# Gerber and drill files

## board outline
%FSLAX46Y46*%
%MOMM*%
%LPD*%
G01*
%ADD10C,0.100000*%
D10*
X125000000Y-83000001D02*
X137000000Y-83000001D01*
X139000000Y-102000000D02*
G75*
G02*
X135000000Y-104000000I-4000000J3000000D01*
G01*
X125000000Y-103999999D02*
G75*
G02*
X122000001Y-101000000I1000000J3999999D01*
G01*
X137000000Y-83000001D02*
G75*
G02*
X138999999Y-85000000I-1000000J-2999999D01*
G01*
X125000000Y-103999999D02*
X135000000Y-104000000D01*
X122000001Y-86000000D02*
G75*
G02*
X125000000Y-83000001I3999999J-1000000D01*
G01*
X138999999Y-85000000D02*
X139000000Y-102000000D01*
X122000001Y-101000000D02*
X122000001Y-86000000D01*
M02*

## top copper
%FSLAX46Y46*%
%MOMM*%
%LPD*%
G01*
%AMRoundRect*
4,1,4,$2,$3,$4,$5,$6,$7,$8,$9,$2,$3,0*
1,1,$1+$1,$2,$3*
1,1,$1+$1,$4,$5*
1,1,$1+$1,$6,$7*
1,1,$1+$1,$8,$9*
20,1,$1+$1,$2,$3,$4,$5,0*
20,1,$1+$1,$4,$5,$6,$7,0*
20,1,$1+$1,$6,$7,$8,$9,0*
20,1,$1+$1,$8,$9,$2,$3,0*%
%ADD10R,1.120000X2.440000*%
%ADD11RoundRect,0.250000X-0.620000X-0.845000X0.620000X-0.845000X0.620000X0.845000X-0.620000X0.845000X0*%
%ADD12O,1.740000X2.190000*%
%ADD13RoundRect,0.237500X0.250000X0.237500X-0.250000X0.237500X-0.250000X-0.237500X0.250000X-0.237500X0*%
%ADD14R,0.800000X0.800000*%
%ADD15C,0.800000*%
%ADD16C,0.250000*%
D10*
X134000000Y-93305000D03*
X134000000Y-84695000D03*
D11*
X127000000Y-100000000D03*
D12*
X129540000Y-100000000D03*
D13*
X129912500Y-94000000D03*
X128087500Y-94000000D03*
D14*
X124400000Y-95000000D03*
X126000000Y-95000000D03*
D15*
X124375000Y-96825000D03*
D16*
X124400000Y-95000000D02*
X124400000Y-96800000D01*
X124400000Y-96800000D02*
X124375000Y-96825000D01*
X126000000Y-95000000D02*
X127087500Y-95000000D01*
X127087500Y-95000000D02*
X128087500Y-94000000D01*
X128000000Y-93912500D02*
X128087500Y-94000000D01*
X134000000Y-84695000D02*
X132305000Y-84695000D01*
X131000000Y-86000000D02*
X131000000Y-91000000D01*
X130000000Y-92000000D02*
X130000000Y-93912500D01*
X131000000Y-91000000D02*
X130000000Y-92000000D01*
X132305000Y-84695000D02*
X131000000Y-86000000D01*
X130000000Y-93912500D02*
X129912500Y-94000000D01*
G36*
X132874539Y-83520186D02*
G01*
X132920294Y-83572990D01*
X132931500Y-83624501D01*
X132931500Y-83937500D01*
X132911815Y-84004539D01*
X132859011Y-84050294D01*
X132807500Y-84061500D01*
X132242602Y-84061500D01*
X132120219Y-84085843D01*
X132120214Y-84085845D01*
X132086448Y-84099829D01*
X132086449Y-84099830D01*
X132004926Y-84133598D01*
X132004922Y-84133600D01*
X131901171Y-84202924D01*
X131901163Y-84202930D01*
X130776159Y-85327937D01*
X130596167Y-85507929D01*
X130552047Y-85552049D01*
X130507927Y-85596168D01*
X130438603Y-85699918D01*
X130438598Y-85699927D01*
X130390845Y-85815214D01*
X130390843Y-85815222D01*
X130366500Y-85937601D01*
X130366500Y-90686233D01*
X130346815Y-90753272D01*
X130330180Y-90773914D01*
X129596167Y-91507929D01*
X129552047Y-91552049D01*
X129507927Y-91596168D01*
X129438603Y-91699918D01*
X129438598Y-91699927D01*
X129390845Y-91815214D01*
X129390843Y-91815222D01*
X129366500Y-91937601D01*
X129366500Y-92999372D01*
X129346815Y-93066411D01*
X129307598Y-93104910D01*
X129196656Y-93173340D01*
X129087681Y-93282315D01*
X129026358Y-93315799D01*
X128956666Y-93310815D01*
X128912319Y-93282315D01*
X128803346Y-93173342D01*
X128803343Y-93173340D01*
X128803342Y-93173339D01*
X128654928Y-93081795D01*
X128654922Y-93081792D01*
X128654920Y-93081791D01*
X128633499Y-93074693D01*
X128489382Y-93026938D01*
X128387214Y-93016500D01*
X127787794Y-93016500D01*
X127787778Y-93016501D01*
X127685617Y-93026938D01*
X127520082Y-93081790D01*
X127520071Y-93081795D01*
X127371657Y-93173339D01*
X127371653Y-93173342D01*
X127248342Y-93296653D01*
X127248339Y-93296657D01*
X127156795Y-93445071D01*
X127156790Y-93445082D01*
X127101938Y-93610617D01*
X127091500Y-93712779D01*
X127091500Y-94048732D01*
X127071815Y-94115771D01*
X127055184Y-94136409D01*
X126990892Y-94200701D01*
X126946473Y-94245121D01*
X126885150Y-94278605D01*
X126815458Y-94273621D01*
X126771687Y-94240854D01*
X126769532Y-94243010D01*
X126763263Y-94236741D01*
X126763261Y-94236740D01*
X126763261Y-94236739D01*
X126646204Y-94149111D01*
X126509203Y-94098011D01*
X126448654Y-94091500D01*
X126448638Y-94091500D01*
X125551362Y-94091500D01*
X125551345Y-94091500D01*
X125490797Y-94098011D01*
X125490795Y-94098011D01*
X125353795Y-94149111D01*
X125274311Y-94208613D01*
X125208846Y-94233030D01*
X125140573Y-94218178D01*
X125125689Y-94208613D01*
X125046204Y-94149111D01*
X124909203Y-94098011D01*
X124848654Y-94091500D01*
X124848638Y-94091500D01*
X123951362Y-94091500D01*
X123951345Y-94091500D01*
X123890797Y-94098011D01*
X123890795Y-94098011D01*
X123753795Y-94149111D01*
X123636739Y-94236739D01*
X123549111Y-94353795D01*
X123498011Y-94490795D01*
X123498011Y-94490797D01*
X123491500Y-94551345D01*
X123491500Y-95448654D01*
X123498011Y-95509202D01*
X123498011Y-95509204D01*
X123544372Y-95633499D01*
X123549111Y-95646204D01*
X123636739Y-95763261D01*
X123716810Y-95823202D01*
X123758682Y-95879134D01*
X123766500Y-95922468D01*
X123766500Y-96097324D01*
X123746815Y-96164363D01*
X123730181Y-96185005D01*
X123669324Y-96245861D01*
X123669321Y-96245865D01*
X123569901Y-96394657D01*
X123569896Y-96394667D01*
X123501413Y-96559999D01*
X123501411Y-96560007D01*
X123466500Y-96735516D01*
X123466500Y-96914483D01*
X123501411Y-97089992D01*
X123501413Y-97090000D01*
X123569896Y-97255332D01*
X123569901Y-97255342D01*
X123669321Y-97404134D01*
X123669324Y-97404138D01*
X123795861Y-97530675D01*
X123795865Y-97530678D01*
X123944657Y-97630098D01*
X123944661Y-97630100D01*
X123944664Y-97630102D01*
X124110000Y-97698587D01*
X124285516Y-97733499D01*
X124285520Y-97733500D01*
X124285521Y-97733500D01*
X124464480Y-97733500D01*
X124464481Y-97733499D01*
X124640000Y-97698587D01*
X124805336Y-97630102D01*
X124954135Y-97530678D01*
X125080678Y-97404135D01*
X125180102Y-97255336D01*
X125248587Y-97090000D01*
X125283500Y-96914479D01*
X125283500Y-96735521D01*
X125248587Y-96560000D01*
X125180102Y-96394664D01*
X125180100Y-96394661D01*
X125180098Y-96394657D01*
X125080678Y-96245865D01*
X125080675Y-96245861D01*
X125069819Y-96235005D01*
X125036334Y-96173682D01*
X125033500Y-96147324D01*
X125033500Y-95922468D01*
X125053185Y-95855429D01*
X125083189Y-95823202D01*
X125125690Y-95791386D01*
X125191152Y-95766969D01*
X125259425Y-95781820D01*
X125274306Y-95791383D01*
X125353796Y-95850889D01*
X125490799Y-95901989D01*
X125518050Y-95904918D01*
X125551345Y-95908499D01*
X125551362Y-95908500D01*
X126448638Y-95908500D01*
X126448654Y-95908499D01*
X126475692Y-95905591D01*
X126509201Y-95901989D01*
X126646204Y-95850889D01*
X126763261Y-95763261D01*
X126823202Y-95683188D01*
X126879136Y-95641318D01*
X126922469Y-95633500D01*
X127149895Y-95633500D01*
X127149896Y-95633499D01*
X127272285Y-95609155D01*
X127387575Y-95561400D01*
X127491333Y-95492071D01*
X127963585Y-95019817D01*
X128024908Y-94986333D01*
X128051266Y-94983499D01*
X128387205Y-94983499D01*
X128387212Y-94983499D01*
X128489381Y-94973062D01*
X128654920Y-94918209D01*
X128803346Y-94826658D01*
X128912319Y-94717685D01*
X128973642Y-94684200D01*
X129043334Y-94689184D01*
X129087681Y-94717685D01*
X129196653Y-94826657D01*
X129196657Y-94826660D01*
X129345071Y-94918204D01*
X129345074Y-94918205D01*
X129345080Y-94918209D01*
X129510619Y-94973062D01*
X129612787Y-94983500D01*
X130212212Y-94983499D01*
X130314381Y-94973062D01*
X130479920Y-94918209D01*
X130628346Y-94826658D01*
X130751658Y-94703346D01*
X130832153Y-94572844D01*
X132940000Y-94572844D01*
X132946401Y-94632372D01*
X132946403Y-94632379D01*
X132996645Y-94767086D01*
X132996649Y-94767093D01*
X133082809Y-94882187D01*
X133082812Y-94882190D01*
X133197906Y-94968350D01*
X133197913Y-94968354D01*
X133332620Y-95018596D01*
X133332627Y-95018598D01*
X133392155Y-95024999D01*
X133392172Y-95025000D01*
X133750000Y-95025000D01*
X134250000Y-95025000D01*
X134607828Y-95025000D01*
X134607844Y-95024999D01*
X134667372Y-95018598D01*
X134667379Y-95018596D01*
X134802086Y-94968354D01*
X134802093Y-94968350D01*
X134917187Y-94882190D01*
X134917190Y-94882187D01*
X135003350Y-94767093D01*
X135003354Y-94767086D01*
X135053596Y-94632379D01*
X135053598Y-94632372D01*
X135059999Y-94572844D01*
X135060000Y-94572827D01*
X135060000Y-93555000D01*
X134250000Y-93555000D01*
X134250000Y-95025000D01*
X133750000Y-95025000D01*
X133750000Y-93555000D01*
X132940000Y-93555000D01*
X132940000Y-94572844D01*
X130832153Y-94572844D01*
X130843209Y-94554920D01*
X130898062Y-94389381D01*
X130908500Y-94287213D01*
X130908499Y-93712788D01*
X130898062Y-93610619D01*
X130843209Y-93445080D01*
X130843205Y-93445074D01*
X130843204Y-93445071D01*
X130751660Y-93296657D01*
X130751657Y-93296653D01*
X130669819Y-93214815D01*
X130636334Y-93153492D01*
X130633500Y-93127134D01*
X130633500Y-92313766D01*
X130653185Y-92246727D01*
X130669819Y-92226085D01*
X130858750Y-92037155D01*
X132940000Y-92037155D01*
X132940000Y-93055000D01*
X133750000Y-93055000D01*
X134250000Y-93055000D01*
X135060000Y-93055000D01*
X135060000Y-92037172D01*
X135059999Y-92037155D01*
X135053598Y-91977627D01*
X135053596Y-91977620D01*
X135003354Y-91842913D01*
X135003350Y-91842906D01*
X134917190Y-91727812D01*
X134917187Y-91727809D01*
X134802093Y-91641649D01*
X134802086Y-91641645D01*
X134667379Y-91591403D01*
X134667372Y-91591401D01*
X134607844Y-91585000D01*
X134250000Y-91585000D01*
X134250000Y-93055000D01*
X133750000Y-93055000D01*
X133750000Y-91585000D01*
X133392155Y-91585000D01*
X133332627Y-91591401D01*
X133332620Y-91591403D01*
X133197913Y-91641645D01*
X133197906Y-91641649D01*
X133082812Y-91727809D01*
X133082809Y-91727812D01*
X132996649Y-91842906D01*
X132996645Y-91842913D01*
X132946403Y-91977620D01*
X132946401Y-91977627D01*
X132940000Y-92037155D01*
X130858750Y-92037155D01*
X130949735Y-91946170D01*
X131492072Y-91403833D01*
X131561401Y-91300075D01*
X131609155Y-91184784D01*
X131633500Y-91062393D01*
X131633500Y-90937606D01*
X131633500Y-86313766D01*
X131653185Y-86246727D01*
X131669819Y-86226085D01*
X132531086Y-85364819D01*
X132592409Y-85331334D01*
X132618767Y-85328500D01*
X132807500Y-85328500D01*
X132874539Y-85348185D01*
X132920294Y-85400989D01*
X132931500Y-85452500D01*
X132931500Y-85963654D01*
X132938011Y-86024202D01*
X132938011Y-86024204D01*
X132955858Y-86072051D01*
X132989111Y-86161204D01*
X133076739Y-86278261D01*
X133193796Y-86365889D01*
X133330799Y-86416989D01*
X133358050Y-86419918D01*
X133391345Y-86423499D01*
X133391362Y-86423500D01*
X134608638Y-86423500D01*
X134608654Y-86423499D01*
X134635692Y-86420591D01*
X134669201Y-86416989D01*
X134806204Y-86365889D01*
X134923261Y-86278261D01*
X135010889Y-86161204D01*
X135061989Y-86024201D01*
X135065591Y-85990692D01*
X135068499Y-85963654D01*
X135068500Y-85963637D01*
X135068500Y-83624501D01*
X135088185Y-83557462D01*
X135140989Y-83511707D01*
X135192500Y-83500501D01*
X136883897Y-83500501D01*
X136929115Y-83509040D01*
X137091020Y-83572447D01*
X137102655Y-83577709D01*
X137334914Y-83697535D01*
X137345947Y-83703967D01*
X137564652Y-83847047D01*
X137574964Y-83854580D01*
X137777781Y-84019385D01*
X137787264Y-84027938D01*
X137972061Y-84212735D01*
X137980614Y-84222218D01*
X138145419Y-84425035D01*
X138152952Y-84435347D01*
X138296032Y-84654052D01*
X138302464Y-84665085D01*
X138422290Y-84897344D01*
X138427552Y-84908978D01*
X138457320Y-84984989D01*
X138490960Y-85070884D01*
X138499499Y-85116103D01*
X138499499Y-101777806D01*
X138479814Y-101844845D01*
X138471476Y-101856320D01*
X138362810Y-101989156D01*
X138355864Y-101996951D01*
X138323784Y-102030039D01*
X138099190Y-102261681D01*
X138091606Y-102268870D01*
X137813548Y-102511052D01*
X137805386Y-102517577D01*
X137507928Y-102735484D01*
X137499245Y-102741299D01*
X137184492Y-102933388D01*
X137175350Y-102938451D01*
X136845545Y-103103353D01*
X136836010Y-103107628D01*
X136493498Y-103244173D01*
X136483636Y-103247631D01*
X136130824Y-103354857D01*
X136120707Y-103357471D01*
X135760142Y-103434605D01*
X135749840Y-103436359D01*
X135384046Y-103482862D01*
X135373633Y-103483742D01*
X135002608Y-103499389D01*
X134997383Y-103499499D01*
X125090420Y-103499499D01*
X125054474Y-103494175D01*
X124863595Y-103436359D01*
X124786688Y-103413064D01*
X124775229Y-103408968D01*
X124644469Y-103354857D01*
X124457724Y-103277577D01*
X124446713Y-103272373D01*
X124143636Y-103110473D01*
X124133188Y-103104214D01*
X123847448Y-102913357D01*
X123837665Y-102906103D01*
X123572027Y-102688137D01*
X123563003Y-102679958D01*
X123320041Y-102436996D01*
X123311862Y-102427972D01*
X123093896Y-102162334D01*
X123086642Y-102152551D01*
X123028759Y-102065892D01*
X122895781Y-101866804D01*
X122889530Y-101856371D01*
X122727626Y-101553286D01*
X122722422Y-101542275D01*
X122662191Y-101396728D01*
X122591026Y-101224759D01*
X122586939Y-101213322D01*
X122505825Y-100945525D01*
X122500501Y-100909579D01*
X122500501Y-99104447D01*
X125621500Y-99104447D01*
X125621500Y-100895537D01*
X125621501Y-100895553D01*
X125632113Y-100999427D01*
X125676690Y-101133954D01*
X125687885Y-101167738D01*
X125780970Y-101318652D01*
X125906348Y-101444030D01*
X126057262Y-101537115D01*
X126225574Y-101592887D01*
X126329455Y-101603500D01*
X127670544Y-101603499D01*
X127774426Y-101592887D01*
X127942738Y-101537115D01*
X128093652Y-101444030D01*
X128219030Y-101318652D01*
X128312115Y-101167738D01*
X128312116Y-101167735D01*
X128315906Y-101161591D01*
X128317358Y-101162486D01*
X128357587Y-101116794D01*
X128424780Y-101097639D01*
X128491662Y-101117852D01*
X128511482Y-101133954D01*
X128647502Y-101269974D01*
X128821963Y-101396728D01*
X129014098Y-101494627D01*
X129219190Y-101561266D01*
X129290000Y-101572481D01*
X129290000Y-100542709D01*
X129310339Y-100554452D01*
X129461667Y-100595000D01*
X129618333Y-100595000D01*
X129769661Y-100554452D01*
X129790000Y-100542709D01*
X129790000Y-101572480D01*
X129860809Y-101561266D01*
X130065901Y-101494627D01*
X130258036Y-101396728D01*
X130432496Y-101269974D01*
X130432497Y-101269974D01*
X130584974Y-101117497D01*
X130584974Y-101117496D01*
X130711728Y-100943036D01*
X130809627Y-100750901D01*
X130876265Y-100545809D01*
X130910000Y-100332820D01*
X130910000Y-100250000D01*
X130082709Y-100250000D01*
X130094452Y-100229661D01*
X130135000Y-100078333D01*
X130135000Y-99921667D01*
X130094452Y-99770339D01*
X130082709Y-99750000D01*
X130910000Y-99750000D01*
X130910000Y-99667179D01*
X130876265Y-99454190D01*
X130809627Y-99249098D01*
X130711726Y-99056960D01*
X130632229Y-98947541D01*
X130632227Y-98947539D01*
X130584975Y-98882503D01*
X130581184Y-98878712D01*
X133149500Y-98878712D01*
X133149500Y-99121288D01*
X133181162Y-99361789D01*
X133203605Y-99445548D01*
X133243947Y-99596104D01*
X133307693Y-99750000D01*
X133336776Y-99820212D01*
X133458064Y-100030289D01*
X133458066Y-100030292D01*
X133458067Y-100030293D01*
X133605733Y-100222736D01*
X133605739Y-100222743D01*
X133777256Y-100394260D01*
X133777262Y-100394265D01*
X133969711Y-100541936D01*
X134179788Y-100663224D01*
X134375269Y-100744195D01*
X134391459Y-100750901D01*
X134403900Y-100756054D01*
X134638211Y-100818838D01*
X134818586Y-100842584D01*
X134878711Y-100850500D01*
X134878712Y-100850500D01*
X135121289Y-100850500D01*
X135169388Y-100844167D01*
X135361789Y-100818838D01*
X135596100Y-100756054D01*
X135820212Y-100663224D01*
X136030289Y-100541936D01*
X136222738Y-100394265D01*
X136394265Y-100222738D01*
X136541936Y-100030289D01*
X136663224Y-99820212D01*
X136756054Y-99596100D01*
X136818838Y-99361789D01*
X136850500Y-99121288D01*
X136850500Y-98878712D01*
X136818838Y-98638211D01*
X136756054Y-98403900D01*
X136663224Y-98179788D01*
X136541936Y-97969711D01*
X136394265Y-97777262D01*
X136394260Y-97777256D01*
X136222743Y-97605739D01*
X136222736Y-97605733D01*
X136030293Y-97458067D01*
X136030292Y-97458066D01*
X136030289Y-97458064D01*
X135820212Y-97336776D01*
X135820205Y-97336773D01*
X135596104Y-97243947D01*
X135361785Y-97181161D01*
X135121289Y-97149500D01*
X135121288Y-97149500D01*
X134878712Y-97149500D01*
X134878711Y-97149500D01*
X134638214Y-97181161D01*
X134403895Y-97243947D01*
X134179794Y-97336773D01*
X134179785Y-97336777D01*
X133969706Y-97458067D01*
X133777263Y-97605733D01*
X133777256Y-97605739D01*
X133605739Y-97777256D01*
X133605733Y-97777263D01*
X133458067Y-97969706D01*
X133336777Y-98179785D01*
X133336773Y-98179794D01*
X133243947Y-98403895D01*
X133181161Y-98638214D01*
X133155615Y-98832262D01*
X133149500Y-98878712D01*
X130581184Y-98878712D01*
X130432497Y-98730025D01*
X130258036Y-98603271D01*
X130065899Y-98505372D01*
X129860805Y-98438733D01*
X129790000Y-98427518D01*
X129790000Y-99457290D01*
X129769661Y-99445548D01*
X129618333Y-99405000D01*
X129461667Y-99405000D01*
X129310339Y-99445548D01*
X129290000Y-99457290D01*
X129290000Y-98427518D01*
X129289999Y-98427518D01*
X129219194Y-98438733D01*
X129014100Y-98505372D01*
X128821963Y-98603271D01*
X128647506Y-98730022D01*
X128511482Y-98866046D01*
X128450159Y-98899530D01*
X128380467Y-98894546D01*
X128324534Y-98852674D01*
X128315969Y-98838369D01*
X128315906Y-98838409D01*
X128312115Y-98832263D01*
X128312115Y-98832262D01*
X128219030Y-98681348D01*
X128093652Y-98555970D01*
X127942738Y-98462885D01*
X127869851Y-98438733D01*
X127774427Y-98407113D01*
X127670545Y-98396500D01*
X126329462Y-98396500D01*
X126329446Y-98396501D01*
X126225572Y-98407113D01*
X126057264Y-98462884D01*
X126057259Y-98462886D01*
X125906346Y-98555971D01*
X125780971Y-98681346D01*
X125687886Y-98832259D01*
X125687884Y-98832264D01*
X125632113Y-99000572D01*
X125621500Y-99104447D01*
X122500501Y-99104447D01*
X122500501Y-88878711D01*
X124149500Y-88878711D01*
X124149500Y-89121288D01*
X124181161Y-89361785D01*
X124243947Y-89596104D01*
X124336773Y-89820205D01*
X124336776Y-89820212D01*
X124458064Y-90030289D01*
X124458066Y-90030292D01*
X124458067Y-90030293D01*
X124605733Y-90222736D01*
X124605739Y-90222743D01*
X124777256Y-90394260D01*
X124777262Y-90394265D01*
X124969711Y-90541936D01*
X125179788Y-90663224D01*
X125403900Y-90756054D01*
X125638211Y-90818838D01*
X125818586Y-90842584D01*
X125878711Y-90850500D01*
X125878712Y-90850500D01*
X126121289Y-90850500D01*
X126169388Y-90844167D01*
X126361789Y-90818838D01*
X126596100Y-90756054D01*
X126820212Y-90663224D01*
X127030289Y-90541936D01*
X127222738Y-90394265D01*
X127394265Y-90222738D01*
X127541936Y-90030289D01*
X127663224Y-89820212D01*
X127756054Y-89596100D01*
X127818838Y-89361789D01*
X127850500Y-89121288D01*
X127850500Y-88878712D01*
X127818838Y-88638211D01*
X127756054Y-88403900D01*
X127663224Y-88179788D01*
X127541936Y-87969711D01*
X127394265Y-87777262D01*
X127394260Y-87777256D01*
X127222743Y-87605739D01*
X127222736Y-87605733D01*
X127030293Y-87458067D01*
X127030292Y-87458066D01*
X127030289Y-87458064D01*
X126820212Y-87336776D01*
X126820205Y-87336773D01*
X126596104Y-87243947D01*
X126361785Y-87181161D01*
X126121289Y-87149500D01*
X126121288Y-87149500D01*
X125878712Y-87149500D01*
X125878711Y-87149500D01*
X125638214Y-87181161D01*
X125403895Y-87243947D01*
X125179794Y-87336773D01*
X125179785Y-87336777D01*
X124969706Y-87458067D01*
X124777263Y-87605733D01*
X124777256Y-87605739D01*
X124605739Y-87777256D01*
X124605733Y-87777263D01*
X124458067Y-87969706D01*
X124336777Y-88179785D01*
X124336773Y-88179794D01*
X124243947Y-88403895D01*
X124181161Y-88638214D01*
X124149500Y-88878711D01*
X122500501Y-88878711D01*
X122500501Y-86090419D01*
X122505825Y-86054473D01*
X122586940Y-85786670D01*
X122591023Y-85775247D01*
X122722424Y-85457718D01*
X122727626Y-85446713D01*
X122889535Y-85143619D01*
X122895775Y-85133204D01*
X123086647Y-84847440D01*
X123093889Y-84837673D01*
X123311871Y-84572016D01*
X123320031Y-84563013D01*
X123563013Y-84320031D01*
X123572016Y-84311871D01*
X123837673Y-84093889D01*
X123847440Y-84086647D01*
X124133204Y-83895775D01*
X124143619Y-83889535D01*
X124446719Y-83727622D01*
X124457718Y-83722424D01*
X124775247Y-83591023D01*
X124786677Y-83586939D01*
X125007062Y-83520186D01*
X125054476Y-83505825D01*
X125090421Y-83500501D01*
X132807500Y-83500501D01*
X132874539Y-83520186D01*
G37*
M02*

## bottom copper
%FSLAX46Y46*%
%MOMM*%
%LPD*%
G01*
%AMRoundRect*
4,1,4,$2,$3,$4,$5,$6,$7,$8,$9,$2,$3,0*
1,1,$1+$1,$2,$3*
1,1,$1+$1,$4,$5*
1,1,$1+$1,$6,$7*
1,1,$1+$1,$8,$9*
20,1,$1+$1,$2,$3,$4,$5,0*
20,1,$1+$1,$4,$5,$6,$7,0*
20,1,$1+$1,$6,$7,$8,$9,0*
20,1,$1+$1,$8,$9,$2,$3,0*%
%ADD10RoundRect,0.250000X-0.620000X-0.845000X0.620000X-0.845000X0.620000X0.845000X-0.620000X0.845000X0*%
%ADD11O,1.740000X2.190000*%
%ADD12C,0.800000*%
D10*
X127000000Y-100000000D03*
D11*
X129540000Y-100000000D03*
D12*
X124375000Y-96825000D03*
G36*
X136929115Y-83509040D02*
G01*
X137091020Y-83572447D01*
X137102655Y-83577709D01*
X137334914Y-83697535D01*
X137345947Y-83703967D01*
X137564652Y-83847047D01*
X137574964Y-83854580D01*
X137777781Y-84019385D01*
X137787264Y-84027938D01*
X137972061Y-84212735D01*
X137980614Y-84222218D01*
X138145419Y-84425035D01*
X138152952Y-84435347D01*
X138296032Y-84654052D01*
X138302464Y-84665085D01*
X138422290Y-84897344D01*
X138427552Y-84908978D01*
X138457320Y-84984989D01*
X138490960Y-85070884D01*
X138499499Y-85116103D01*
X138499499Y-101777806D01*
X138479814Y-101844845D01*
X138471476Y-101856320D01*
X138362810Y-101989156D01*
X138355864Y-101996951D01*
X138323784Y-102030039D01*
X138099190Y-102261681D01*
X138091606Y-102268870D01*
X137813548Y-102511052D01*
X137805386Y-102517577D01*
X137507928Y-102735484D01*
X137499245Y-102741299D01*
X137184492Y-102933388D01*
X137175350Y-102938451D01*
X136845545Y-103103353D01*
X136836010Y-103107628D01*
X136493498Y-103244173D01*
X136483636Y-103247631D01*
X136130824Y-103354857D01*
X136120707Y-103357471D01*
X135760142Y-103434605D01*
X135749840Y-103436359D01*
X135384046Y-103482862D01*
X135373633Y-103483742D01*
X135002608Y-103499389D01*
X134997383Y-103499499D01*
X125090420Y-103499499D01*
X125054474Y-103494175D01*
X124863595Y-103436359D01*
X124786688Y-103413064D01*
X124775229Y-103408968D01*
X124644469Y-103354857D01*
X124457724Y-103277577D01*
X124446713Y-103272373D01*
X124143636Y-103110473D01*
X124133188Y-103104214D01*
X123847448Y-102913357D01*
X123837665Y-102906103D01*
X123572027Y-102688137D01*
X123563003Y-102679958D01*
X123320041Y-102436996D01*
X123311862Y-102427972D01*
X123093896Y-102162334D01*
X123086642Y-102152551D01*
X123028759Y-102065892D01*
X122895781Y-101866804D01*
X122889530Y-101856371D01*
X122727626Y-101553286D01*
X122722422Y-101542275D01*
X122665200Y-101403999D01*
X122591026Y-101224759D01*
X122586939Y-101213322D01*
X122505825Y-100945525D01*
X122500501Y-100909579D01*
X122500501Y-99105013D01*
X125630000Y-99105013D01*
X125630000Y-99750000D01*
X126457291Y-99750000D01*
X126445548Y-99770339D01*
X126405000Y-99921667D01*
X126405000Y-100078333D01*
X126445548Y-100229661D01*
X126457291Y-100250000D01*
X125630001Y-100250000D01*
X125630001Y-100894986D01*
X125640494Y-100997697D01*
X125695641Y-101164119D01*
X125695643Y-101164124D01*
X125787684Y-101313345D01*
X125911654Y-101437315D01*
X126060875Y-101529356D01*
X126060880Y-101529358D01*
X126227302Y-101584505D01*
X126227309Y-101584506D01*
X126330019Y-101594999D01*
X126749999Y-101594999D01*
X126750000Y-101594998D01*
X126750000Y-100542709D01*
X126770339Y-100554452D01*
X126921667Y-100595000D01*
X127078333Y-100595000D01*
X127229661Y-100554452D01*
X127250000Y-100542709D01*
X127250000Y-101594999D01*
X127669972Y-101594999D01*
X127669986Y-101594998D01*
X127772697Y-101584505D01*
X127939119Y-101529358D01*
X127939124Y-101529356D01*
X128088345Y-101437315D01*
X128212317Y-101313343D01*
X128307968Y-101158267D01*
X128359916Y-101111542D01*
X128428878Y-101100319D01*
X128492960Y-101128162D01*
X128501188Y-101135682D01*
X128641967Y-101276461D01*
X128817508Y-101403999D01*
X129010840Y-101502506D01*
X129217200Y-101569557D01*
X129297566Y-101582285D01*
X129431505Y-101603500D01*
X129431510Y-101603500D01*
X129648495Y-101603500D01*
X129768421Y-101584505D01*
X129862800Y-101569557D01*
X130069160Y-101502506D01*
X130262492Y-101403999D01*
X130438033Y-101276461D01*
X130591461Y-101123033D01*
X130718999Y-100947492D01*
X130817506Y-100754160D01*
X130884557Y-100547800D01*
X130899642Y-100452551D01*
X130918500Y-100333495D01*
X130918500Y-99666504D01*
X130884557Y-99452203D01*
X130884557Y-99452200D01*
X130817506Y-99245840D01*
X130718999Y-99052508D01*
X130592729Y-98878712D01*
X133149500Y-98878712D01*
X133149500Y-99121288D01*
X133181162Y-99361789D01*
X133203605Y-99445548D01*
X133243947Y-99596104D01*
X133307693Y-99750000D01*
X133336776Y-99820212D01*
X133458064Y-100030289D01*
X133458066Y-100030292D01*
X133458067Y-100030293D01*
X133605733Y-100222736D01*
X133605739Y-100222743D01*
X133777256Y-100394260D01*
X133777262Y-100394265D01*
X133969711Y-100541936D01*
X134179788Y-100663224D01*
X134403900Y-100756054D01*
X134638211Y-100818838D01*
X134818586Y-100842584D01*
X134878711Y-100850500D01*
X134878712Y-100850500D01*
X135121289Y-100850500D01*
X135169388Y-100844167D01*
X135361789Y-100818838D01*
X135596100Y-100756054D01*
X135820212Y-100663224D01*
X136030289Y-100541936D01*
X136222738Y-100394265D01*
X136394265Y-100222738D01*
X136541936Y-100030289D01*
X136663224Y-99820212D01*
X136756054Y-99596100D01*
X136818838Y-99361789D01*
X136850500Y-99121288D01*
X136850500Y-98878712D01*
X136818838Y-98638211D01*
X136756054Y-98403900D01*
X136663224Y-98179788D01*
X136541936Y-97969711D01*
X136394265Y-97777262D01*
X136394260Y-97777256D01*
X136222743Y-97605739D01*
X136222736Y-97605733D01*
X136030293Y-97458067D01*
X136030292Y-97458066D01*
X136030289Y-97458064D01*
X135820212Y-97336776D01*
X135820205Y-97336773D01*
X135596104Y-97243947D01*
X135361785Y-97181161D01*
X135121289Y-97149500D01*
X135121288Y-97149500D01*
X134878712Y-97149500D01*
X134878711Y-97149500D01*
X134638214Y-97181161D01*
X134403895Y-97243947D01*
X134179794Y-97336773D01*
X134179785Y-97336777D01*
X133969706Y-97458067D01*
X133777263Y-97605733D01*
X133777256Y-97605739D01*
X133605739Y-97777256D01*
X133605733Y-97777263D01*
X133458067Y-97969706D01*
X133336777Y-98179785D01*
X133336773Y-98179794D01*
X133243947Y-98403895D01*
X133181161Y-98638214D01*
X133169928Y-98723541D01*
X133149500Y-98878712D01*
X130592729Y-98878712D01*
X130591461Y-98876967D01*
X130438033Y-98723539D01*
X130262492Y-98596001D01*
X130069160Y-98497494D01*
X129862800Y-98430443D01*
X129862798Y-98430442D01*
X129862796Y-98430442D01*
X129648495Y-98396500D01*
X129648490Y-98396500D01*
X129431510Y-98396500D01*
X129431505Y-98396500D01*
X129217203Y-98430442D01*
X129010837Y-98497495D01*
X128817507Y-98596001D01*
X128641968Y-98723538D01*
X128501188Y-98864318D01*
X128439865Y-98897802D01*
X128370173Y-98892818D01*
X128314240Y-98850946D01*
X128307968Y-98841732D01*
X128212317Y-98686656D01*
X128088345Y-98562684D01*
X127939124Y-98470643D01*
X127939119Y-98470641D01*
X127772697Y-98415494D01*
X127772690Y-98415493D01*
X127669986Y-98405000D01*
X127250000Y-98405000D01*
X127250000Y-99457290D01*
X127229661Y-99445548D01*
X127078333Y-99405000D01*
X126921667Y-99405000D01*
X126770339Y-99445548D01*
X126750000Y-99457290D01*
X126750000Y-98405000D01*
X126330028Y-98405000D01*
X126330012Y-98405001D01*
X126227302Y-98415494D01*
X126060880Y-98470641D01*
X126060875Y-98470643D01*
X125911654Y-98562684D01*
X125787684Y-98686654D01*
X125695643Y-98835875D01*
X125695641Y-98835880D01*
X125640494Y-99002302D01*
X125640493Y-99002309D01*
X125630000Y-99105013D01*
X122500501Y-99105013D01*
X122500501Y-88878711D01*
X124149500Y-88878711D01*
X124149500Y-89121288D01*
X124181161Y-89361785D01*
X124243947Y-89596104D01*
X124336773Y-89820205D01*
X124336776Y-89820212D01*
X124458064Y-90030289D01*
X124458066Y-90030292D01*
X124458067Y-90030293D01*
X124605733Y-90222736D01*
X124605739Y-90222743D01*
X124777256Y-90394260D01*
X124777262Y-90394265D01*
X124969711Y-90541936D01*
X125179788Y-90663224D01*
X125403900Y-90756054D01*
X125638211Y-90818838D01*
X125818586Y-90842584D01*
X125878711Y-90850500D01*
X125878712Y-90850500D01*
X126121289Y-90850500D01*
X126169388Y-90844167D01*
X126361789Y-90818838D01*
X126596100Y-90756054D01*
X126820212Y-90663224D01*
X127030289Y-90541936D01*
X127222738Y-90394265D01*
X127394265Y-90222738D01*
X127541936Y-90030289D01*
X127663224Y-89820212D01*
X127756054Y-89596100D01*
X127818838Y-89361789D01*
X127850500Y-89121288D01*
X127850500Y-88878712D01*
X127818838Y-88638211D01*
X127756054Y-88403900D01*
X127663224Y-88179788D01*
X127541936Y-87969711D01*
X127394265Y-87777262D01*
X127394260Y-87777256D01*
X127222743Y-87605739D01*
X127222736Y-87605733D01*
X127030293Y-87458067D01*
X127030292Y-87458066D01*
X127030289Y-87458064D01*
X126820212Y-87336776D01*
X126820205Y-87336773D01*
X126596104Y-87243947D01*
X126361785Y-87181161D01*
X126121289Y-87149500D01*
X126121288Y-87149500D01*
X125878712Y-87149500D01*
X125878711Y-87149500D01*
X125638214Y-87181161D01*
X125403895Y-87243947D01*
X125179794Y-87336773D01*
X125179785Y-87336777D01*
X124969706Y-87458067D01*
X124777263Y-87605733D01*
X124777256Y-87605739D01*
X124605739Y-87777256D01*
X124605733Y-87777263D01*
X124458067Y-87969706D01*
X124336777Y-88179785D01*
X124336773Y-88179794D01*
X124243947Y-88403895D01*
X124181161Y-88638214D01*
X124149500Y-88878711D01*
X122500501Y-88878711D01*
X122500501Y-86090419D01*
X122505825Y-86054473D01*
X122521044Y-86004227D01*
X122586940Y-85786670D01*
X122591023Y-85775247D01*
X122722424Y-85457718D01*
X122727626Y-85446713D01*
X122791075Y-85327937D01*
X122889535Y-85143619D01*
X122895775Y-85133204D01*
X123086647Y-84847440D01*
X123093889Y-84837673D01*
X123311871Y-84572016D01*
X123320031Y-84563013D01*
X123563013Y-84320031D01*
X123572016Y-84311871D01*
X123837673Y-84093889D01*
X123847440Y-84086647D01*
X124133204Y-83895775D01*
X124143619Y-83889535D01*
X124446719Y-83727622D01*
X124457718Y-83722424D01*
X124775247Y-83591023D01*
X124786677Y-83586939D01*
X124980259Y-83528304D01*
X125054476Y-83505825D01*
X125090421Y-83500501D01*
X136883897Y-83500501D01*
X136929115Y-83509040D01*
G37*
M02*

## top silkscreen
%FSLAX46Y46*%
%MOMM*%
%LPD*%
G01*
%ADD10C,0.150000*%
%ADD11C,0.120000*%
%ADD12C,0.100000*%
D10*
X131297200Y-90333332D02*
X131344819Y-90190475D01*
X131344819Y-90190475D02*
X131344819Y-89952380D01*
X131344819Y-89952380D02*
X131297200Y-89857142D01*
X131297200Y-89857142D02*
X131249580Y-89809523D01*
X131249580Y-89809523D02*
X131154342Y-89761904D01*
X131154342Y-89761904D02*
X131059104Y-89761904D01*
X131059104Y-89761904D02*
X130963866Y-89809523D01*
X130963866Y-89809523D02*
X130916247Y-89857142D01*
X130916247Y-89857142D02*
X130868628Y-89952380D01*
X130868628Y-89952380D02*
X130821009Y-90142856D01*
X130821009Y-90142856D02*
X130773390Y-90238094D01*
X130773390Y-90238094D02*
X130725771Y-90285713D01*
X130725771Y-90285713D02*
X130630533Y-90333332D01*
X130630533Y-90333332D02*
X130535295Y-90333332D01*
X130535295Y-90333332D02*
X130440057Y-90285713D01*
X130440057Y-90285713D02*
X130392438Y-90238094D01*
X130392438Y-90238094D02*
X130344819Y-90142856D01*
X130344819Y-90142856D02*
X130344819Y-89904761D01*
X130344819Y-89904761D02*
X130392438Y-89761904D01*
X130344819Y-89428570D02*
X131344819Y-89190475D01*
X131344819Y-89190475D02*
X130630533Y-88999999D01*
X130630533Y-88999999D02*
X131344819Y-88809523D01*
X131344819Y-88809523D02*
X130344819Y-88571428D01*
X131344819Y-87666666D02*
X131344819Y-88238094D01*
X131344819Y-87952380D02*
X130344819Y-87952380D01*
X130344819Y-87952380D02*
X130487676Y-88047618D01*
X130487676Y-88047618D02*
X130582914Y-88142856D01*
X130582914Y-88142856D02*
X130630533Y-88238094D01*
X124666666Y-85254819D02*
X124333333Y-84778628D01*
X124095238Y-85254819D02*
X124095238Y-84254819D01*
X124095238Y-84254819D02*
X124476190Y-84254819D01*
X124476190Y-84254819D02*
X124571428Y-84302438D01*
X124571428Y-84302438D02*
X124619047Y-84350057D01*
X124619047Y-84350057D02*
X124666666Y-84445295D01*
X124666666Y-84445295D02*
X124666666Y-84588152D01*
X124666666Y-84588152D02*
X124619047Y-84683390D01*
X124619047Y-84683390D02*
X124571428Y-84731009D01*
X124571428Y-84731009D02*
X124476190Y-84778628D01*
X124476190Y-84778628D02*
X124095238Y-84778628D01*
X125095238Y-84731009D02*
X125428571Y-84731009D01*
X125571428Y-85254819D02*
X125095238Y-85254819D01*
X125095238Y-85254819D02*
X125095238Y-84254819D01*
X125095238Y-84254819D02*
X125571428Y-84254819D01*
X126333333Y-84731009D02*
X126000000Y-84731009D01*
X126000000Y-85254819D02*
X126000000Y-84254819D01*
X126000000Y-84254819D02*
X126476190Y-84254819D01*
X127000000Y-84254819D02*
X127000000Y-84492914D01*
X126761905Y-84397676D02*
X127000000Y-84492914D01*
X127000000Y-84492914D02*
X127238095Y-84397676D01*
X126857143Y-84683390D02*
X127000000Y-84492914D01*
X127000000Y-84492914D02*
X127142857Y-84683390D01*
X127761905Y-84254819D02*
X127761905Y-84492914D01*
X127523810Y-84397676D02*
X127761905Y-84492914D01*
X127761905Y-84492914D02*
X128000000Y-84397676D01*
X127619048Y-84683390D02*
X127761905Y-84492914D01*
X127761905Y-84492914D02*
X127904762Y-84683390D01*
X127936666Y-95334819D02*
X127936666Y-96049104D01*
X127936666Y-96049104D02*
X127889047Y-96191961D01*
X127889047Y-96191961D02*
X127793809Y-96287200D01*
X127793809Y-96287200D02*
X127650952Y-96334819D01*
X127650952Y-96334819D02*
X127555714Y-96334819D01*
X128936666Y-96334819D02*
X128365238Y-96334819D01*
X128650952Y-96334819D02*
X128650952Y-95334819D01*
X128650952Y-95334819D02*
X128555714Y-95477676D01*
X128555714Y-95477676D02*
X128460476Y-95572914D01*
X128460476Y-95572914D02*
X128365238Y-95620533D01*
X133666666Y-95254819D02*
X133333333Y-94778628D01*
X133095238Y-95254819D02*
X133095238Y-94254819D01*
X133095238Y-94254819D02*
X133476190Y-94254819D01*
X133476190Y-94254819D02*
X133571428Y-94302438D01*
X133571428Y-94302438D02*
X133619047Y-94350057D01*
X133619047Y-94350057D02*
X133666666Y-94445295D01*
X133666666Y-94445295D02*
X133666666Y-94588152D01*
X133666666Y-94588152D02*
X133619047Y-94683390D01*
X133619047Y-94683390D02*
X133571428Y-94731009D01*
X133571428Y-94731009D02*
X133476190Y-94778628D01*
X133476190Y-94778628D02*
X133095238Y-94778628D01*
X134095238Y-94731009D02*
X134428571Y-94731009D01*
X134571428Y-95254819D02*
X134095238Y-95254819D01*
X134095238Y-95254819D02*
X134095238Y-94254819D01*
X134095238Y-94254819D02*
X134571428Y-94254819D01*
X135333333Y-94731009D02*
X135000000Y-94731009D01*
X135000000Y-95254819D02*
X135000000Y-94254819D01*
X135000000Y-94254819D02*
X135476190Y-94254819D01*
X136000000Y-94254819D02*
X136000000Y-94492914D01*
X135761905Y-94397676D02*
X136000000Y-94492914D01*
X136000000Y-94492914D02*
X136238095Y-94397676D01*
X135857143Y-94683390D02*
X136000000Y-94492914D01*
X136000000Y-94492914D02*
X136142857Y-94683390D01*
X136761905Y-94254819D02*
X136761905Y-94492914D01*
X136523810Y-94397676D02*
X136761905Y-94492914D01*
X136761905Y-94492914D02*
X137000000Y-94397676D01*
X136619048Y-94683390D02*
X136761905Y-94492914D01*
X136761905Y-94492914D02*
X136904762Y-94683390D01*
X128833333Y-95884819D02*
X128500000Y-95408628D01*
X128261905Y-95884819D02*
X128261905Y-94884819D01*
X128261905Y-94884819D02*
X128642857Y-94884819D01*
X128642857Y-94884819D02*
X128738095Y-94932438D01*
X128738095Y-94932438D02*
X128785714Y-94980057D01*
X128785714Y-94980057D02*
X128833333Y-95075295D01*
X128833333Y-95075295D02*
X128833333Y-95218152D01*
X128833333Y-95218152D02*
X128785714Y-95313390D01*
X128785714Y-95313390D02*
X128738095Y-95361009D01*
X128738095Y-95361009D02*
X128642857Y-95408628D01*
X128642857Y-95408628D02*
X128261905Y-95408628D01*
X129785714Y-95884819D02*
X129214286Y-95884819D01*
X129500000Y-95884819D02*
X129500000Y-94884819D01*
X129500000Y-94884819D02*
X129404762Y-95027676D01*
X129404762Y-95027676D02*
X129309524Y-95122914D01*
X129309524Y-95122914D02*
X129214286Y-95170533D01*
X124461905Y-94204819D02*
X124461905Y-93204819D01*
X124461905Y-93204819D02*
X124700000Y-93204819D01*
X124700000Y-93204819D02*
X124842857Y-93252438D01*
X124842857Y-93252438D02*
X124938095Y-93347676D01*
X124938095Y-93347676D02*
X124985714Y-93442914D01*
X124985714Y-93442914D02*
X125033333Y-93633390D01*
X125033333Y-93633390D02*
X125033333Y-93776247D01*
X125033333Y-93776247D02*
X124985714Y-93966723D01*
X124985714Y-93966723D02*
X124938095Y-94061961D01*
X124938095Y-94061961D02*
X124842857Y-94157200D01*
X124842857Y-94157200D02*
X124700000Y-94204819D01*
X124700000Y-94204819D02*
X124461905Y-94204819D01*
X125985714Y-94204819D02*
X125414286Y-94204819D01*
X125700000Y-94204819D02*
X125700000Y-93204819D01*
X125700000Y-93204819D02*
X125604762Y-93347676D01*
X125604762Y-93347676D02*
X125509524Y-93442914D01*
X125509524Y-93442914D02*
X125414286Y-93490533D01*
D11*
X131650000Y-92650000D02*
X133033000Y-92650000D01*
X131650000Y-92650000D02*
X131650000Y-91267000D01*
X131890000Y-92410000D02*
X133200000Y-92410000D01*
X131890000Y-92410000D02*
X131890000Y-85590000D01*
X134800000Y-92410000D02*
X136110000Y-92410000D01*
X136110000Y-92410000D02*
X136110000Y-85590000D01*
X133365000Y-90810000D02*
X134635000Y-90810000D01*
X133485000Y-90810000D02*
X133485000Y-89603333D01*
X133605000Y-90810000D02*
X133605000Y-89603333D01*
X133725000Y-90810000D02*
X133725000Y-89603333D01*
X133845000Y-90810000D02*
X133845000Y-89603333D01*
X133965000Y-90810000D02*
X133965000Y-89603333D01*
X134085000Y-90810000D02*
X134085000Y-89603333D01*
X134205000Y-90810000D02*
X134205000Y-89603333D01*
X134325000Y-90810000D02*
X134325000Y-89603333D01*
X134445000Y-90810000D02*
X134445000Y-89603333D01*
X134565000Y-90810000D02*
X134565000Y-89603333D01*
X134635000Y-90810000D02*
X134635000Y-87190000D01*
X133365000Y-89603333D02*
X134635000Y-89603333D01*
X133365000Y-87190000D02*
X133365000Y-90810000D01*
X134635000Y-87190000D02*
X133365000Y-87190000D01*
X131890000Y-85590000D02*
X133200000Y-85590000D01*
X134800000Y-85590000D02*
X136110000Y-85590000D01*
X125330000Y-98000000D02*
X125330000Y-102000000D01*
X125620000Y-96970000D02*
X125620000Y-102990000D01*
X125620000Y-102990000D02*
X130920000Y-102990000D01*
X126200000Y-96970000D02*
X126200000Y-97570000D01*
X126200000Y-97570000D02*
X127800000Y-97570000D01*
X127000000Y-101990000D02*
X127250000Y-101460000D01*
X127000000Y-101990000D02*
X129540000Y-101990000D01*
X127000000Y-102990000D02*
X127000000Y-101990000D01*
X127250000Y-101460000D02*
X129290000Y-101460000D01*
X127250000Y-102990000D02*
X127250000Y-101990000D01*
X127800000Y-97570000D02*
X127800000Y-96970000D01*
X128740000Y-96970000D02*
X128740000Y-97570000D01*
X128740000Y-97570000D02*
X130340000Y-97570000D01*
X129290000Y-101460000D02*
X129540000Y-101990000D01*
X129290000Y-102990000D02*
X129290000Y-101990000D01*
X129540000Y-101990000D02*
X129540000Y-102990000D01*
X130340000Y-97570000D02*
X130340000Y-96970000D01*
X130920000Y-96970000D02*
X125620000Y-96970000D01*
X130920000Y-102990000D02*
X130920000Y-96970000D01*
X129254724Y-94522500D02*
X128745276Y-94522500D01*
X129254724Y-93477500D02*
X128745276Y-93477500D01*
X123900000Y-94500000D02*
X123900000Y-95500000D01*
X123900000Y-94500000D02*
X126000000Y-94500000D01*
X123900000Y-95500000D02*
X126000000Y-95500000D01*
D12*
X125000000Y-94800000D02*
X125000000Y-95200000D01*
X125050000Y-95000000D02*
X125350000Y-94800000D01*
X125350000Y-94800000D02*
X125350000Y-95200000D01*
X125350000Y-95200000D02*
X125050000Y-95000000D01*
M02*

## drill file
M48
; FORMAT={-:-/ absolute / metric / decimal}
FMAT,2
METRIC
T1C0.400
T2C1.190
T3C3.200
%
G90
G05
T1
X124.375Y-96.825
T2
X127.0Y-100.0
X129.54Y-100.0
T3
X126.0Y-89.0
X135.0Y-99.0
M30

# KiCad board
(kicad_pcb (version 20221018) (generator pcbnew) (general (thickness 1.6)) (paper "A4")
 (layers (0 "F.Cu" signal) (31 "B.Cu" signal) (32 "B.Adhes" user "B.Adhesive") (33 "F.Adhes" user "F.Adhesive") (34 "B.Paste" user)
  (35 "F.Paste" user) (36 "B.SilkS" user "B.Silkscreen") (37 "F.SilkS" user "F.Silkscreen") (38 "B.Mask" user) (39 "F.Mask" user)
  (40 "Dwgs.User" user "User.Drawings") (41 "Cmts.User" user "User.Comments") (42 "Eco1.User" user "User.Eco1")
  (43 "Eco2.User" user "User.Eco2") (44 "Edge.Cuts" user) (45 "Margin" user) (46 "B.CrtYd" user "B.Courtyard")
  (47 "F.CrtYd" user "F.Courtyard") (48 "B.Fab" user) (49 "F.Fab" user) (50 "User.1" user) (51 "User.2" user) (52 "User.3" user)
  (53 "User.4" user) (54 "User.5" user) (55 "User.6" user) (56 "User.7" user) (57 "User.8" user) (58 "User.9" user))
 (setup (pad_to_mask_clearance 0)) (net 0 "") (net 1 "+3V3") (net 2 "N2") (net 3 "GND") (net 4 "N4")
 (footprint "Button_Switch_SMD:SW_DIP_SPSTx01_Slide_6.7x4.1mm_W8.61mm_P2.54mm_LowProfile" (layer "F.Cu") (at 134 89 90)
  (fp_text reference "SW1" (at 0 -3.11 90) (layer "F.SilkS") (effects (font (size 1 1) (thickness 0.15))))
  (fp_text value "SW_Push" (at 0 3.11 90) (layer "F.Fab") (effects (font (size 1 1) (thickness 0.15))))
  (fp_line (start -3.65 -2.35) (end -3.65 -0.967) (stroke (width 0.12) (type solid)) (layer "F.SilkS"))
  (fp_line (start -3.65 -2.35) (end -2.267 -2.35) (stroke (width 0.12) (type solid)) (layer "F.SilkS"))
  (fp_line (start -3.41 -2.11) (end -3.41 -0.8) (stroke (width 0.12) (type solid)) (layer "F.SilkS"))
  (fp_line (start -3.41 -2.11) (end 3.41 -2.11) (stroke (width 0.12) (type solid)) (layer "F.SilkS"))
  (fp_line (start -3.41 0.8) (end -3.41 2.11) (stroke (width 0.12) (type solid)) (layer "F.SilkS"))
  (fp_line (start -3.41 2.11) (end 3.41 2.11) (stroke (width 0.12) (type solid)) (layer "F.SilkS"))
  (fp_line (start -1.81 -0.635) (end -1.81 0.635) (stroke (width 0.12) (type solid)) (layer "F.SilkS"))
  (fp_line (start -1.81 -0.515) (end -0.603333 -0.515) (stroke (width 0.12) (type solid)) (layer "F.SilkS"))
  (fp_line (start -1.81 -0.395) (end -0.603333 -0.395) (stroke (width 0.12) (type solid)) (layer "F.SilkS"))
  (fp_line (start -1.81 -0.275) (end -0.603333 -0.275) (stroke (width 0.12) (type solid)) (layer "F.SilkS"))
  (fp_line (start -1.81 -0.155) (end -0.603333 -0.155) (stroke (width 0.12) (type solid)) (layer "F.SilkS"))
  (fp_line (start -1.81 -0.035) (end -0.603333 -0.035) (stroke (width 0.12) (type solid)) (layer "F.SilkS"))
  (fp_line (start -1.81 0.085) (end -0.603333 0.085) (stroke (width 0.12) (type solid)) (layer "F.SilkS"))
  (fp_line (start -1.81 0.205) (end -0.603333 0.205) (stroke (width 0.12) (type solid)) (layer "F.SilkS"))
  (fp_line (start -1.81 0.325) (end -0.603333 0.325) (stroke (width 0.12) (type solid)) (layer "F.SilkS"))
  (fp_line (start -1.81 0.445) (end -0.603333 0.445) (stroke (width 0.12) (type solid)) (layer "F.SilkS"))
  (fp_line (start -1.81 0.565) (end -0.603333 0.565) (stroke (width 0.12) (type solid)) (layer "F.SilkS"))
  (fp_line (start -1.81 0.635) (end 1.81 0.635) (stroke (width 0.12) (type solid)) (layer "F.SilkS"))
  (fp_line (start -0.603333 -0.635) (end -0.603333 0.635) (stroke (width 0.12) (type solid)) (layer "F.SilkS"))
  (fp_line (start 1.81 -0.635) (end -1.81 -0.635) (stroke (width 0.12) (type solid)) (layer "F.SilkS"))
  (fp_line (start 1.81 0.635) (end 1.81 -0.635) (stroke (width 0.12) (type solid)) (layer "F.SilkS"))
  (fp_line (start 3.41 -2.11) (end 3.41 -0.8) (stroke (width 0.12) (type solid)) (layer "F.SilkS"))
  (fp_line (start 3.41 0.8) (end 3.41 2.11) (stroke (width 0.12) (type solid)) (layer "F.SilkS"))
  (pad "1" smd rect (at -4.305 0 90) (size 2.44 1.12) (layers "F.Cu" "F.Paste" "F.Mask") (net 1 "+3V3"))
  (pad "2" smd rect (at 4.305 0 90) (size 2.44 1.12) (layers "F.Cu" "F.Paste" "F.Mask") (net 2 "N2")))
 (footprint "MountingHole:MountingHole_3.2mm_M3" (layer "F.Cu") (at 126 89)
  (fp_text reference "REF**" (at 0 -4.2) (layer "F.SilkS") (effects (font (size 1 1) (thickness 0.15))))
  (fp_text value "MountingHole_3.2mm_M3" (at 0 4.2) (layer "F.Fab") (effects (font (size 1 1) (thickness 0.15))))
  (pad "" np_thru_hole circle (at 0 0) (size 3.2 3.2) (drill 3.2) (layers "*.Cu" "*.Mask")))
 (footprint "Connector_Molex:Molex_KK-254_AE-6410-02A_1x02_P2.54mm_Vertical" (layer "F.Cu") (at 127 100)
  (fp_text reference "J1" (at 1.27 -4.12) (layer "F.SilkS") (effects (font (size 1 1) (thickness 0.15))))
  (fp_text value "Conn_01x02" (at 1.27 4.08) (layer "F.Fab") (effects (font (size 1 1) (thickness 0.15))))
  (fp_line (start -1.67 -2) (end -1.67 2) (stroke (width 0.12) (type solid)) (layer "F.SilkS"))
  (fp_line (start -1.38 -3.03) (end -1.38 2.99) (stroke (width 0.12) (type solid)) (layer "F.SilkS"))
  (fp_line (start -1.38 2.99) (end 3.92 2.99) (stroke (width 0.12) (type solid)) (layer "F.SilkS"))
  (fp_line (start -0.8 -3.03) (end -0.8 -2.43) (stroke (width 0.12) (type solid)) (layer "F.SilkS"))
  (fp_line (start -0.8 -2.43) (end 0.8 -2.43) (stroke (width 0.12) (type solid)) (layer "F.SilkS"))
  (fp_line (start 0 1.99) (end 0.25 1.46) (stroke (width 0.12) (type solid)) (layer "F.SilkS"))
  (fp_line (start 0 1.99) (end 2.54 1.99) (stroke (width 0.12) (type solid)) (layer "F.SilkS"))
  (fp_line (start 0 2.99) (end 0 1.99) (stroke (width 0.12) (type solid)) (layer "F.SilkS"))
  (fp_line (start 0.25 1.46) (end 2.29 1.46) (stroke (width 0.12) (type solid)) (layer "F.SilkS"))
  (fp_line (start 0.25 2.99) (end 0.25 1.99) (stroke (width 0.12) (type solid)) (layer "F.SilkS"))
  (fp_line (start 0.8 -2.43) (end 0.8 -3.03) (stroke (width 0.12) (type solid)) (layer "F.SilkS"))
  (fp_line (start 1.74 -3.03) (end 1.74 -2.43) (stroke (width 0.12) (type solid)) (layer "F.SilkS"))
  (fp_line (start 1.74 -2.43) (end 3.34 -2.43) (stroke (width 0.12) (type solid)) (layer "F.SilkS"))
  (fp_line (start 2.29 1.46) (end 2.54 1.99) (stroke (width 0.12) (type solid)) (layer "F.SilkS"))
  (fp_line (start 2.29 2.99) (end 2.29 1.99) (stroke (width 0.12) (type solid)) (layer "F.SilkS"))
  (fp_line (start 2.54 1.99) (end 2.54 2.99) (stroke (width 0.12) (type solid)) (layer "F.SilkS"))
  (fp_line (start 3.34 -2.43) (end 3.34 -3.03) (stroke (width 0.12) (type solid)) (layer "F.SilkS"))
  (fp_line (start 3.92 -3.03) (end -1.38 -3.03) (stroke (width 0.12) (type solid)) (layer "F.SilkS"))
  (fp_line (start 3.92 2.99) (end 3.92 -3.03) (stroke (width 0.12) (type solid)) (layer "F.SilkS"))
  (pad "1" thru_hole roundrect (at 0 0) (size 1.74 2.19) (drill 1.19) (layers "*.Cu" "*.Mask") (roundrect_rratio 0.143678) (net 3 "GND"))
  (pad "2" thru_hole oval (at 2.54 0) (size 1.74 2.19) (drill 1.19) (layers "*.Cu" "*.Mask") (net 1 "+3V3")))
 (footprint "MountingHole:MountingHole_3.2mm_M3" (layer "F.Cu") (at 135 99)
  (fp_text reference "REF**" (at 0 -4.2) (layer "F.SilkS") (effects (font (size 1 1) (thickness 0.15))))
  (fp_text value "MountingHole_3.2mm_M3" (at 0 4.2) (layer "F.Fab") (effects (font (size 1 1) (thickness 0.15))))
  (pad "" np_thru_hole circle (at 0 0) (size 3.2 3.2) (drill 3.2) (layers "*.Cu" "*.Mask")))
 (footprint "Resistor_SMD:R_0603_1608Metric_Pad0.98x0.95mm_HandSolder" (layer "F.Cu") (at 129 94 180)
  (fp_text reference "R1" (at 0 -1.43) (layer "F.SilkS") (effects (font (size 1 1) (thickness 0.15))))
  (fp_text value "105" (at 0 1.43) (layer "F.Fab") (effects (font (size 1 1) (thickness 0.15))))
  (fp_line (start -0.254724 -0.5225) (end 0.254724 -0.5225) (stroke (width 0.12) (type solid)) (layer "F.SilkS"))
  (fp_line (start -0.254724 0.5225) (end 0.254724 0.5225) (stroke (width 0.12) (type solid)) (layer "F.SilkS"))
  (pad "1" smd roundrect (at -0.9125 0 180) (size 0.975 0.95) (layers "F.Cu" "F.Paste" "F.Mask") (roundrect_rratio 0.25) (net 2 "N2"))
  (pad "2" smd roundrect (at 0.9125 0 180) (size 0.975 0.95) (layers "F.Cu" "F.Paste" "F.Mask") (roundrect_rratio 0.25) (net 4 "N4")))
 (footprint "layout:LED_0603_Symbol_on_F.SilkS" (layer "F.Cu") (at 125.2 95)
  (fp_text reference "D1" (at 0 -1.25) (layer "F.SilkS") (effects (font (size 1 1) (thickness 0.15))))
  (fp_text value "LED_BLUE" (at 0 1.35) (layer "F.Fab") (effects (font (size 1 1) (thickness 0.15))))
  (fp_line (start -1.3 -0.5) (end -1.3 0.5) (stroke (width 0.12) (type solid)) (layer "F.SilkS"))
  (fp_line (start -1.3 -0.5) (end 0.8 -0.5) (stroke (width 0.12) (type solid)) (layer "F.SilkS"))
  (fp_line (start -1.3 0.5) (end 0.8 0.5) (stroke (width 0.12) (type solid)) (layer "F.SilkS"))
  (fp_line (start -0.2 -0.2) (end -0.2 0.2) (stroke (width 0.1) (type solid)) (layer "F.SilkS"))
  (fp_line (start -0.15 0) (end 0.15 -0.2) (stroke (width 0.1) (type solid)) (layer "F.SilkS"))
  (fp_line (start 0.15 -0.2) (end 0.15 0.2) (stroke (width 0.1) (type solid)) (layer "F.SilkS"))
  (fp_line (start 0.15 0.2) (end -0.15 0) (stroke (width 0.1) (type solid)) (layer "F.SilkS"))
  (pad "1" smd rect (at -0.8 0 180) (size 0.8 0.8) (layers "F.Cu" "F.Paste" "F.Mask") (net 3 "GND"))
  (pad "2" smd rect (at 0.8 0 180) (size 0.8 0.8) (layers "F.Cu" "F.Paste" "F.Mask") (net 4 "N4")))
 (gr_line (start 125 83.000001) (end 137 83.000001) (stroke (width 0.1) (type default)) (layer "Edge.Cuts"))
 (gr_arc (start 139 102) (mid 137.236068 103.472136) (end 135 104) (stroke (width 0.1) (type default)) (layer "Edge.Cuts"))
 (gr_arc (start 125 103.999999) (mid 123.084525 102.915475) (end 122.000001 101) (stroke (width 0.1) (type default)) (layer "Edge.Cuts"))
 (gr_arc (start 137 83.000001) (mid 138.236067 83.763933) (end 138.999999 85) (stroke (width 0.1) (type default)) (layer "Edge.Cuts"))
 (gr_line (start 125 103.999999) (end 135 104) (stroke (width 0.1) (type default)) (layer "Edge.Cuts"))
 (gr_arc (start 122.000001 86) (mid 123.084525 84.084525) (end 125 83.000001) (stroke (width 0.1) (type default)) (layer "Edge.Cuts"))
 (gr_line (start 138.999999 85) (end 139 102) (stroke (width 0.1) (type default)) (layer "Edge.Cuts"))
 (gr_line (start 122.000001 101) (end 122.000001 86) (stroke (width 0.1) (type default)) (layer "Edge.Cuts"))
 (segment (start 124.4 95) (end 124.4 96.8) (width 0.25) (layer "F.Cu") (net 3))
 (segment (start 124.4 96.8) (end 124.375 96.825) (width 0.25) (layer "F.Cu") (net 3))
 (via (at 124.375 96.825) (size 0.8) (drill 0.4) (layers "F.Cu" "B.Cu") (free) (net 3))
 (segment (start 126 95) (end 127.0875 95) (width 0.25) (layer "F.Cu") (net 4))
 (segment (start 127.0875 95) (end 128.0875 94) (width 0.25) (layer "F.Cu") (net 4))
 (segment (start 128 93.9125) (end 128.0875 94) (width 0.25) (layer "F.Cu") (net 4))
 (segment (start 134 84.695) (end 132.305 84.695) (width 0.25) (layer "F.Cu") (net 2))
 (segment (start 131 86) (end 131 91) (width 0.25) (layer "F.Cu") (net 2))
 (segment (start 130 92) (end 130 93.9125) (width 0.25) (layer "F.Cu") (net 2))
 (segment (start 131 91) (end 130 92) (width 0.25) (layer "F.Cu") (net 2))
 (segment (start 132.305 84.695) (end 131 86) (width 0.25) (layer "F.Cu") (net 2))
 (segment (start 130 93.9125) (end 129.9125 94) (width 0.25) (layer "F.Cu") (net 2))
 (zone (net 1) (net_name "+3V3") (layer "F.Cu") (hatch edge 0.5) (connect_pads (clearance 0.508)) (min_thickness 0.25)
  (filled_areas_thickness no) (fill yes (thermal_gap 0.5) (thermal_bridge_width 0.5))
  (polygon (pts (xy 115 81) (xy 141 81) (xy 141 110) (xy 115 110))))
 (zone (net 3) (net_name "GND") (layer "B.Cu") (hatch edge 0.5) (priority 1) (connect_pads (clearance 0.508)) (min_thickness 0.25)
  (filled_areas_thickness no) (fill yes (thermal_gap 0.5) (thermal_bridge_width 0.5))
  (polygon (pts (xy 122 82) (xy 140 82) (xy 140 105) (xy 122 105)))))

